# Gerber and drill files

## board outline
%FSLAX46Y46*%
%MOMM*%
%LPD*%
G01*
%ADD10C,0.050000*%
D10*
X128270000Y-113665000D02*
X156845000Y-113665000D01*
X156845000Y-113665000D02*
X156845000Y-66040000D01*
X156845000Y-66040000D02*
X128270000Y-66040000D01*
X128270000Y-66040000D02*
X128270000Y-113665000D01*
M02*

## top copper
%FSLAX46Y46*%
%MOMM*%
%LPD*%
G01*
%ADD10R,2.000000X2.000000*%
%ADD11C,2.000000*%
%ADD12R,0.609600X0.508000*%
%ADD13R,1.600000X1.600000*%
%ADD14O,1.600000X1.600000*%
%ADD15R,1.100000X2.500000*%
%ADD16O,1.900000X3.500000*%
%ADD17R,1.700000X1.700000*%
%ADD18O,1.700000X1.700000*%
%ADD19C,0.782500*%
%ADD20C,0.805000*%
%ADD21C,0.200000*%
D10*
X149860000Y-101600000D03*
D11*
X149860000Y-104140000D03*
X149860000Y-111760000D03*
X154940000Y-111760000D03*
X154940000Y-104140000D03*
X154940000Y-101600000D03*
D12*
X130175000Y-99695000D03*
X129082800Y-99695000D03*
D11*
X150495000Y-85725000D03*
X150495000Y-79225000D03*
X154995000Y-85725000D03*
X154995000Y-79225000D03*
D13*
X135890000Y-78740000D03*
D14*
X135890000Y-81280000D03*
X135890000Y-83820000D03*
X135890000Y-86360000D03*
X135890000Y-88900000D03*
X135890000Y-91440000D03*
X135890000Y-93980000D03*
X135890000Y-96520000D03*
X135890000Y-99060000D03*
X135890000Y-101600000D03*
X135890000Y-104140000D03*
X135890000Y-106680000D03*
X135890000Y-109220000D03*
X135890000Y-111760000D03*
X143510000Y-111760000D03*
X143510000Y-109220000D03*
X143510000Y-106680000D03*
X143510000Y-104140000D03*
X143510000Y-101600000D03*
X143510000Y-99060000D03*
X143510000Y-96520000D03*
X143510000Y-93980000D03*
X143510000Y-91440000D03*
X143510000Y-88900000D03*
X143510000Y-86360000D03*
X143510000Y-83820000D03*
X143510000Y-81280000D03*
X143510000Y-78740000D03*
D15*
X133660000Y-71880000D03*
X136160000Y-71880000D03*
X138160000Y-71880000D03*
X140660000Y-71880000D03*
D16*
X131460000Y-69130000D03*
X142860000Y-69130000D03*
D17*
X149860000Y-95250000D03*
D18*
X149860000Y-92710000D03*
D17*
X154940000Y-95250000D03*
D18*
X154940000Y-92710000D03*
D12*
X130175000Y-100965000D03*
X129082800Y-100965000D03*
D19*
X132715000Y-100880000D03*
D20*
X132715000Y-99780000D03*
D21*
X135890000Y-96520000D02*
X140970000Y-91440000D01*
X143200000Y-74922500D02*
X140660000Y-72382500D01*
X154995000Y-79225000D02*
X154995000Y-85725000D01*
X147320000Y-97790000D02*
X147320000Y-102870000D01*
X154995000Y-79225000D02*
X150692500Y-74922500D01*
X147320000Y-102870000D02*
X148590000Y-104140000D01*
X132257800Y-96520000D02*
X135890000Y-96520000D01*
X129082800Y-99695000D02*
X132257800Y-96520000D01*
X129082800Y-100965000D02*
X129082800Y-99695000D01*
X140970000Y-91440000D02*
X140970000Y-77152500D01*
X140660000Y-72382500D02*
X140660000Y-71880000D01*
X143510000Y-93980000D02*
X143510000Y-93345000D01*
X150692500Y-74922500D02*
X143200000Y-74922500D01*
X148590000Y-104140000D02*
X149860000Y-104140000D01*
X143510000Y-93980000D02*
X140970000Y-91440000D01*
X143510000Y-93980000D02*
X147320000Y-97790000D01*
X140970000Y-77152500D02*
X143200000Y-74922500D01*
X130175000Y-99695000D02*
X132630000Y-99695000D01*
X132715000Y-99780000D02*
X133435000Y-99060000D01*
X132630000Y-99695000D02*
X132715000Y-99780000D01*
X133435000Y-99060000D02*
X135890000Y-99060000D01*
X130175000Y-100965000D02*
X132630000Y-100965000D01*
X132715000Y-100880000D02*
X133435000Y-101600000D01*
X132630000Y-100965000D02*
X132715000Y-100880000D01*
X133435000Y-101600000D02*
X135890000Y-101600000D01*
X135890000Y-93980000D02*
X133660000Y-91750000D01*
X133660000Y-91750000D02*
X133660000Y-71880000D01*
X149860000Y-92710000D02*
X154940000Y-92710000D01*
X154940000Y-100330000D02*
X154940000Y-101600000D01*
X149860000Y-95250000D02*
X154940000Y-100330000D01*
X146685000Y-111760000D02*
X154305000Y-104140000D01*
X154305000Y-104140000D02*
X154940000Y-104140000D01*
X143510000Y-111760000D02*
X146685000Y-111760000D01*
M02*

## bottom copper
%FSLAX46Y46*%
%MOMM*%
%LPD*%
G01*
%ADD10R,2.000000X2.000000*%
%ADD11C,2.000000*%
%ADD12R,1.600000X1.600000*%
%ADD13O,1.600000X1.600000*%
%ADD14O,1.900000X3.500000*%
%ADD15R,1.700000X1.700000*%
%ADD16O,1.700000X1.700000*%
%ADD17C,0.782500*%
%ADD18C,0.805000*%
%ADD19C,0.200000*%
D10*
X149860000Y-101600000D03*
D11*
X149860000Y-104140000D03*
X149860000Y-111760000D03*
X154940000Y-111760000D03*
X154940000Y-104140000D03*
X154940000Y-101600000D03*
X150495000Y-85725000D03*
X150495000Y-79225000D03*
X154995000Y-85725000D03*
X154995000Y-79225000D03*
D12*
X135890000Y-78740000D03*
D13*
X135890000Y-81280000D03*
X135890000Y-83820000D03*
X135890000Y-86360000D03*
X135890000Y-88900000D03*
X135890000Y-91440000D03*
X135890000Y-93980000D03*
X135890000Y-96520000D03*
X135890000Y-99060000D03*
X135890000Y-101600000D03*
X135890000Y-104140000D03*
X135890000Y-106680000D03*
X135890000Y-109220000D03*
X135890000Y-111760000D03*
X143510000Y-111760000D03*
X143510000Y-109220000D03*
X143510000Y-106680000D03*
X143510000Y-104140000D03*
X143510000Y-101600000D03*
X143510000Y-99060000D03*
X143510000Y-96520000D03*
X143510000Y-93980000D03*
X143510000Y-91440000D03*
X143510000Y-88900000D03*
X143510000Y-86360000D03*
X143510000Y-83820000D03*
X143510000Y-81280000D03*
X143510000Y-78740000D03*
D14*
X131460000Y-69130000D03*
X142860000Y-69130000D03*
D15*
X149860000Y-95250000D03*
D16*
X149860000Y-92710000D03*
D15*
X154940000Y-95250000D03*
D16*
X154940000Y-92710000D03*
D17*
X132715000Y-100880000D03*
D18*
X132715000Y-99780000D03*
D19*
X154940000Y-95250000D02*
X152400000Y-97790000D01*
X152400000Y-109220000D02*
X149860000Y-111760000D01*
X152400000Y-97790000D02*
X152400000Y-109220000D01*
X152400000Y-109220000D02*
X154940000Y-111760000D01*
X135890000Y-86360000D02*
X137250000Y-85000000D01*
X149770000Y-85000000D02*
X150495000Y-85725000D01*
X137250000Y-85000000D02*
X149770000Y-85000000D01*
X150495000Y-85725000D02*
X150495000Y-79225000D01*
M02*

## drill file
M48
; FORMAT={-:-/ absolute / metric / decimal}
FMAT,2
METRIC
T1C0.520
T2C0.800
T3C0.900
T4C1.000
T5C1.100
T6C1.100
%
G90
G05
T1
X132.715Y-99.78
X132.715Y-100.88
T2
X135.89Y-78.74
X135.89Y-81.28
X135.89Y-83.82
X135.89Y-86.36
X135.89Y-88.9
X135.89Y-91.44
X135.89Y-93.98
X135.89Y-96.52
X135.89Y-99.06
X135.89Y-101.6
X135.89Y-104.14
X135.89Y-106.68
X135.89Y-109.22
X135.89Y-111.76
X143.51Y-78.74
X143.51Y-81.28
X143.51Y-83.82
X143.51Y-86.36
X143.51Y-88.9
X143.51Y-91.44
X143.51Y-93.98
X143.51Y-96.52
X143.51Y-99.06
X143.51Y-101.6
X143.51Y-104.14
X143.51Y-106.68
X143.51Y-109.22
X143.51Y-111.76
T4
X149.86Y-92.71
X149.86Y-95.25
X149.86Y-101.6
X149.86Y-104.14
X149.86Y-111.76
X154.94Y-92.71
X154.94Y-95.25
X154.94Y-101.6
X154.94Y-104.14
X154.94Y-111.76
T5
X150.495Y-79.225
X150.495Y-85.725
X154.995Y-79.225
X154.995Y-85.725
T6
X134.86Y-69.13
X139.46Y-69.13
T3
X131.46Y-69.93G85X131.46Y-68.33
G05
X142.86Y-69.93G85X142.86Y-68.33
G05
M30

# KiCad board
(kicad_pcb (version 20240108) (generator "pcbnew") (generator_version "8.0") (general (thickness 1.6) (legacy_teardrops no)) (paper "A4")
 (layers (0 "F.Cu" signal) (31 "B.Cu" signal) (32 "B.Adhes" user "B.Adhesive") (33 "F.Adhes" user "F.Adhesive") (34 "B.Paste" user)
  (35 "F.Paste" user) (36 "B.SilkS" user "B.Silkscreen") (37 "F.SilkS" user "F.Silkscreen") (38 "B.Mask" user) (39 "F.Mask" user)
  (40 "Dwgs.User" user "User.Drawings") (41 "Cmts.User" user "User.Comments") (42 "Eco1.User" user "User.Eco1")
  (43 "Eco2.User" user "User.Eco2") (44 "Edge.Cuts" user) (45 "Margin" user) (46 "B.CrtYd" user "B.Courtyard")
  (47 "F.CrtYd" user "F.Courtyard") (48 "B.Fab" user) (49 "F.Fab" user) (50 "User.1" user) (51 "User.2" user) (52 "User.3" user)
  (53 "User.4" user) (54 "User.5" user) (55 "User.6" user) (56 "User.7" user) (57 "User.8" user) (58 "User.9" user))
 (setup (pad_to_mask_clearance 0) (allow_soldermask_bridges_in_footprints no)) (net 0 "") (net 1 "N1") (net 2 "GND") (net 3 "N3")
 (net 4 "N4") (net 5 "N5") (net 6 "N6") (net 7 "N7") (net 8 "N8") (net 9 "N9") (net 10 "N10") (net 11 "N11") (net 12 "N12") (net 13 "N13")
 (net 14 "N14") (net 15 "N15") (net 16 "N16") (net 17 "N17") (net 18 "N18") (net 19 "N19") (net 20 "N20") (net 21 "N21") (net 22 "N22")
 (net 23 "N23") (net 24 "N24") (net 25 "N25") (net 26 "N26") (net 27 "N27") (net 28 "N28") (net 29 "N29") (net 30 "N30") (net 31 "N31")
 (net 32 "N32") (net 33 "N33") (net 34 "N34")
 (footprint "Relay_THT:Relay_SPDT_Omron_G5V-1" (layer "F.Cu") (at 149.86 101.6)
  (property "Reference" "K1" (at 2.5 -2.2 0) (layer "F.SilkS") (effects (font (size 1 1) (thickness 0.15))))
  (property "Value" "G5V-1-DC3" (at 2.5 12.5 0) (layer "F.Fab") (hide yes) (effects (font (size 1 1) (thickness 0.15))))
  (pad "1" thru_hole rect (at 0 0) (size 2 2) (drill 1) (layers "*.Cu" "*.Mask") (remove_unused_layers no) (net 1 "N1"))
  (pad "2" thru_hole circle (at 0 2.54) (size 2 2) (drill 1) (layers "*.Cu" "*.Mask") (remove_unused_layers no) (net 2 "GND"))
  (pad "5" thru_hole circle (at 0 10.16) (size 2 2) (drill 1) (layers "*.Cu" "*.Mask") (remove_unused_layers no) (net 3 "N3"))
  (pad "6" thru_hole circle (at 5.08 10.16) (size 2 2) (drill 1) (layers "*.Cu" "*.Mask") (remove_unused_layers no) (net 3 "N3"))
  (pad "9" thru_hole circle (at 5.08 2.54) (size 2 2) (drill 1) (layers "*.Cu" "*.Mask") (remove_unused_layers no) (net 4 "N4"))
  (pad "10" thru_hole circle (at 5.08 0) (size 2 2) (drill 1) (layers "*.Cu" "*.Mask") (remove_unused_layers no) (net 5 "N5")))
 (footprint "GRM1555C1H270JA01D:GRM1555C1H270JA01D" (layer "F.Cu") (at 129.6289 99.695 180)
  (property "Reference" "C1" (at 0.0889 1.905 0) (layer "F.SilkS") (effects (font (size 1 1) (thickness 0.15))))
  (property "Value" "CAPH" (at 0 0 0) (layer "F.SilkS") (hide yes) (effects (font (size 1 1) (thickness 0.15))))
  (pad "1" smd rect (at -0.5461 0 180) (size 0.6096 0.508) (layers "F.Cu" "F.Paste" "F.Mask") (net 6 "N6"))
  (pad "2" smd rect (at 0.5461 0 180) (size 0.6096 0.508) (layers "F.Cu" "F.Paste" "F.Mask") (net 2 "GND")))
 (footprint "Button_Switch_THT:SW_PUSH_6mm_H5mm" (layer "F.Cu") (at 150.495 85.725 90)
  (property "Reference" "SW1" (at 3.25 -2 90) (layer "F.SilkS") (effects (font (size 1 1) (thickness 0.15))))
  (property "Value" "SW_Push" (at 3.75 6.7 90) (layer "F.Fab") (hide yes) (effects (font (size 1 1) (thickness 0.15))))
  (pad "1" thru_hole circle (at 0 0 180) (size 2 2) (drill 1.1) (layers "*.Cu" "*.Mask") (remove_unused_layers no) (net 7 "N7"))
  (pad "1" thru_hole circle (at 6.5 0 180) (size 2 2) (drill 1.1) (layers "*.Cu" "*.Mask") (remove_unused_layers no) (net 7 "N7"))
  (pad "2" thru_hole circle (at 0 4.5 180) (size 2 2) (drill 1.1) (layers "*.Cu" "*.Mask") (remove_unused_layers no) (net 2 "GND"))
  (pad "2" thru_hole circle (at 6.5 4.5 180) (size 2 2) (drill 1.1) (layers "*.Cu" "*.Mask") (remove_unused_layers no) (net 2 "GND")))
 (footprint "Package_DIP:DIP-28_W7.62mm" (layer "F.Cu") (at 135.89 78.74)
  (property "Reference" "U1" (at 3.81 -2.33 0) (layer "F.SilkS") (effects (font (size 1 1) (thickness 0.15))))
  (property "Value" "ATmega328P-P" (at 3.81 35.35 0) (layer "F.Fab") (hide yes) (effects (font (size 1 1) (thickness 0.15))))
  (pad "1" thru_hole rect (at 0 0) (size 1.6 1.6) (drill 0.8) (layers "*.Cu" "*.Mask") (remove_unused_layers no) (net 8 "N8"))
  (pad "2" thru_hole oval (at 0 2.54) (size 1.6 1.6) (drill 0.8) (layers "*.Cu" "*.Mask") (remove_unused_layers no) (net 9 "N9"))
  (pad "3" thru_hole oval (at 0 5.08) (size 1.6 1.6) (drill 0.8) (layers "*.Cu" "*.Mask") (remove_unused_layers no) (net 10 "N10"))
  (pad "4" thru_hole oval (at 0 7.62) (size 1.6 1.6) (drill 0.8) (layers "*.Cu" "*.Mask") (remove_unused_layers no) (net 7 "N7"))
  (pad "5" thru_hole oval (at 0 10.16) (size 1.6 1.6) (drill 0.8) (layers "*.Cu" "*.Mask") (remove_unused_layers no) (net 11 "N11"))
  (pad "6" thru_hole oval (at 0 12.7) (size 1.6 1.6) (drill 0.8) (layers "*.Cu" "*.Mask") (remove_unused_layers no) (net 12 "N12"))
  (pad "7" thru_hole oval (at 0 15.24) (size 1.6 1.6) (drill 0.8) (layers "*.Cu" "*.Mask") (remove_unused_layers no) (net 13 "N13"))
  (pad "8" thru_hole oval (at 0 17.78) (size 1.6 1.6) (drill 0.8) (layers "*.Cu" "*.Mask") (remove_unused_layers no) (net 2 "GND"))
  (pad "9" thru_hole oval (at 0 20.32) (size 1.6 1.6) (drill 0.8) (layers "*.Cu" "*.Mask") (remove_unused_layers no) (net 6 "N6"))
  (pad "10" thru_hole oval (at 0 22.86) (size 1.6 1.6) (drill 0.8) (layers "*.Cu" "*.Mask") (remove_unused_layers no) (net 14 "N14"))
  (pad "11" thru_hole oval (at 0 25.4) (size 1.6 1.6) (drill 0.8) (layers "*.Cu" "*.Mask") (remove_unused_layers no) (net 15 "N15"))
  (pad "12" thru_hole oval (at 0 27.94) (size 1.6 1.6) (drill 0.8) (layers "*.Cu" "*.Mask") (remove_unused_layers no) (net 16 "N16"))
  (pad "13" thru_hole oval (at 0 30.48) (size 1.6 1.6) (drill 0.8) (layers "*.Cu" "*.Mask") (remove_unused_layers no) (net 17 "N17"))
  (pad "14" thru_hole oval (at 0 33.02) (size 1.6 1.6) (drill 0.8) (layers "*.Cu" "*.Mask") (remove_unused_layers no) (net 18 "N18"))
  (pad "15" thru_hole oval (at 7.62 33.02) (size 1.6 1.6) (drill 0.8) (layers "*.Cu" "*.Mask") (remove_unused_layers no) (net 4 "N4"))
  (pad "16" thru_hole oval (at 7.62 30.48) (size 1.6 1.6) (drill 0.8) (layers "*.Cu" "*.Mask") (remove_unused_layers no) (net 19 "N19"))
  (pad "17" thru_hole oval (at 7.62 27.94) (size 1.6 1.6) (drill 0.8) (layers "*.Cu" "*.Mask") (remove_unused_layers no) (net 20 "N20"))
  (pad "18" thru_hole oval (at 7.62 25.4) (size 1.6 1.6) (drill 0.8) (layers "*.Cu" "*.Mask") (remove_unused_layers no) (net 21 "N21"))
  (pad "19" thru_hole oval (at 7.62 22.86) (size 1.6 1.6) (drill 0.8) (layers "*.Cu" "*.Mask") (remove_unused_layers no) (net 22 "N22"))
  (pad "20" thru_hole oval (at 7.62 20.32) (size 1.6 1.6) (drill 0.8) (layers "*.Cu" "*.Mask") (remove_unused_layers no) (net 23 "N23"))
  (pad "21" thru_hole oval (at 7.62 17.78) (size 1.6 1.6) (drill 0.8) (layers "*.Cu" "*.Mask") (remove_unused_layers no) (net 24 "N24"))
  (pad "22" thru_hole oval (at 7.62 15.24) (size 1.6 1.6) (drill 0.8) (layers "*.Cu" "*.Mask") (remove_unused_layers no) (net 2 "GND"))
  (pad "23" thru_hole oval (at 7.62 12.7) (size 1.6 1.6) (drill 0.8) (layers "*.Cu" "*.Mask") (remove_unused_layers no) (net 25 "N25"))
  (pad "24" thru_hole oval (at 7.62 10.16) (size 1.6 1.6) (drill 0.8) (layers "*.Cu" "*.Mask") (remove_unused_layers no) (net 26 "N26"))
  (pad "25" thru_hole oval (at 7.62 7.62) (size 1.6 1.6) (drill 0.8) (layers "*.Cu" "*.Mask") (remove_unused_layers no) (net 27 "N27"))
  (pad "26" thru_hole oval (at 7.62 5.08) (size 1.6 1.6) (drill 0.8) (layers "*.Cu" "*.Mask") (remove_unused_layers no) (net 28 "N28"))
  (pad "27" thru_hole oval (at 7.62 2.54) (size 1.6 1.6) (drill 0.8) (layers "*.Cu" "*.Mask") (remove_unused_layers no) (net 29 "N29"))
  (pad "28" thru_hole oval (at 7.62 0) (size 1.6 1.6) (drill 0.8) (layers "*.Cu" "*.Mask") (remove_unused_layers no) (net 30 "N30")))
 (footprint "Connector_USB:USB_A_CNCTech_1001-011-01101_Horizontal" (layer "F.Cu") (at 137.16 62.23 90)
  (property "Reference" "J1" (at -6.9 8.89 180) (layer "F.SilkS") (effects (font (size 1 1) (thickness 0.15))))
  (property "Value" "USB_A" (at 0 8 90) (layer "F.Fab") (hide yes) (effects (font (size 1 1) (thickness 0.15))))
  (pad "" np_thru_hole circle (at -6.9 -2.3 90) (size 1.1 1.1) (drill 1.1) (layers "*.Cu" "*.Mask"))
  (pad "" np_thru_hole circle (at -6.9 2.3 90) (size 1.1 1.1) (drill 1.1) (layers "*.Cu" "*.Mask"))
  (pad "1" smd rect (at -9.65 -3.5 90) (size 2.5 1.1) (layers "F.Cu" "F.Paste" "F.Mask") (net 13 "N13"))
  (pad "2" smd rect (at -9.65 -1 90) (size 2.5 1.1) (layers "F.Cu" "F.Paste" "F.Mask") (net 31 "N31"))
  (pad "3" smd rect (at -9.65 1 90) (size 2.5 1.1) (layers "F.Cu" "F.Paste" "F.Mask") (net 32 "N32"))
  (pad "4" smd rect (at -9.65 3.5 90) (size 2.5 1.1) (layers "F.Cu" "F.Paste" "F.Mask") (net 2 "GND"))
  (pad "5" thru_hole oval (at -6.9 -5.7 90) (size 3.5 1.9) (drill oval 2.5 0.9) (layers "*.Cu" "*.Mask") (remove_unused_layers no)
   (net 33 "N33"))
  (pad "5" thru_hole oval (at -6.9 5.7 90) (size 3.5 1.9) (drill oval 2.5 0.9) (layers "*.Cu" "*.Mask") (remove_unused_layers no)
   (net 33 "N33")))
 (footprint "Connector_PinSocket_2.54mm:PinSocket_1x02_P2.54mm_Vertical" (layer "F.Cu") (at 149.86 95.25 180)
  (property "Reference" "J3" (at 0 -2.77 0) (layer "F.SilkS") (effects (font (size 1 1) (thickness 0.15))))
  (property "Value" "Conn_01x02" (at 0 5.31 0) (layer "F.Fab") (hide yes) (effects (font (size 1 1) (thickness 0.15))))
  (pad "1" thru_hole rect (at 0 0 180) (size 1.7 1.7) (drill 1) (layers "*.Cu" "*.Mask") (remove_unused_layers no) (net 5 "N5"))
  (pad "2" thru_hole oval (at 0 2.54 180) (size 1.7 1.7) (drill 1) (layers "*.Cu" "*.Mask") (remove_unused_layers no) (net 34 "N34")))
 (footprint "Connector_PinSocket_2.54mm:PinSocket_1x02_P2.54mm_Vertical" (layer "F.Cu") (at 154.94 95.25 180)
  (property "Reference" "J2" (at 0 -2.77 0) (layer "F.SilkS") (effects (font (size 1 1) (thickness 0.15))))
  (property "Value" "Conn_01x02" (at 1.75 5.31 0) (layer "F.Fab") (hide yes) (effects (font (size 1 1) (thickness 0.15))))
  (pad "1" thru_hole rect (at 0 0 180) (size 1.7 1.7) (drill 1) (layers "*.Cu" "*.Mask") (remove_unused_layers no) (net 3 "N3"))
  (pad "2" thru_hole oval (at 0 2.54 180) (size 1.7 1.7) (drill 1) (layers "*.Cu" "*.Mask") (remove_unused_layers no) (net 34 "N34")))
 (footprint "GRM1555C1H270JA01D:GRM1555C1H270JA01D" (layer "F.Cu") (at 129.6289 100.965 180)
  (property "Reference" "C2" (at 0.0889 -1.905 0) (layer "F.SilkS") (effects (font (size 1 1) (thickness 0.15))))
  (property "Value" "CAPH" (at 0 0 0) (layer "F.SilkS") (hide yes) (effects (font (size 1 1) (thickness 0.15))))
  (pad "1" smd rect (at -0.5461 0 180) (size 0.6096 0.508) (layers "F.Cu" "F.Paste" "F.Mask") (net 14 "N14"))
  (pad "2" smd rect (at 0.5461 0 180) (size 0.6096 0.508) (layers "F.Cu" "F.Paste" "F.Mask") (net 2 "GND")))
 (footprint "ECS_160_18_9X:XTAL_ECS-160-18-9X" (layer "F.Cu") (at 132.715 100.33 90)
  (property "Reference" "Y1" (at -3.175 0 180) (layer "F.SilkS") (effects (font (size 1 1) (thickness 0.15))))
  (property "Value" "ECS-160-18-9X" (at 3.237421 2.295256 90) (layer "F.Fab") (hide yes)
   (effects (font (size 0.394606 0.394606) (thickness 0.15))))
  (pad "1" thru_hole circle (at -0.55 0 90) (size 0.7825 0.7825) (drill 0.52) (layers "*.Cu" "*.Mask") (remove_unused_layers no)
   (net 14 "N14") (solder_mask_margin 0.102))
  (pad "2" thru_hole circle (at 0.55 0 90) (size 0.805 0.805) (drill 0.52) (layers "*.Cu" "*.Mask") (remove_unused_layers no) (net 6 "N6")
   (solder_mask_margin 0.102)))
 (gr_line (start 128.27 113.665) (end 156.845 113.665) (stroke (width 0.05) (type default)) (layer "Edge.Cuts"))
 (gr_line (start 156.845 113.665) (end 156.845 66.04) (stroke (width 0.05) (type default)) (layer "Edge.Cuts"))
 (gr_line (start 156.845 66.04) (end 128.27 66.04) (stroke (width 0.05) (type default)) (layer "Edge.Cuts"))
 (gr_line (start 128.27 66.04) (end 128.27 113.665) (stroke (width 0.05) (type default)) (layer "Edge.Cuts"))
 (segment (start 135.89 96.52) (end 140.97 91.44) (width 0.2) (layer "F.Cu") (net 2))
 (segment (start 143.2 74.9225) (end 140.66 72.3825) (width 0.2) (layer "F.Cu") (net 2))
 (segment (start 154.995 79.225) (end 154.995 85.725) (width 0.2) (layer "F.Cu") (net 2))
 (segment (start 147.32 97.79) (end 147.32 102.87) (width 0.2) (layer "F.Cu") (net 2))
 (segment (start 154.995 79.225) (end 150.6925 74.9225) (width 0.2) (layer "F.Cu") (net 2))
 (segment (start 147.32 102.87) (end 148.59 104.14) (width 0.2) (layer "F.Cu") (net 2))
 (segment (start 132.2578 96.52) (end 135.89 96.52) (width 0.2) (layer "F.Cu") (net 2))
 (segment (start 129.0828 99.695) (end 132.2578 96.52) (width 0.2) (layer "F.Cu") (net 2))
 (segment (start 129.0828 100.965) (end 129.0828 99.695) (width 0.2) (layer "F.Cu") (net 2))
 (segment (start 140.97 91.44) (end 140.97 77.1525) (width 0.2) (layer "F.Cu") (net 2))
 (segment (start 140.66 72.3825) (end 140.66 71.88) (width 0.2) (layer "F.Cu") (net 2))
 (segment (start 143.51 93.98) (end 143.51 93.345) (width 0.2) (layer "F.Cu") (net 2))
 (segment (start 150.6925 74.9225) (end 143.2 74.9225) (width 0.2) (layer "F.Cu") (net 2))
 (segment (start 148.59 104.14) (end 149.86 104.14) (width 0.2) (layer "F.Cu") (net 2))
 (segment (start 143.51 93.98) (end 140.97 91.44) (width 0.2) (layer "F.Cu") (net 2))
 (segment (start 143.51 93.98) (end 147.32 97.79) (width 0.2) (layer "F.Cu") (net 2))
 (segment (start 140.97 77.1525) (end 143.2 74.9225) (width 0.2) (layer "F.Cu") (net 2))
 (segment (start 130.175 99.695) (end 132.63 99.695) (width 0.2) (layer "F.Cu") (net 6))
 (segment (start 132.715 99.78) (end 133.435 99.06) (width 0.2) (layer "F.Cu") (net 6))
 (segment (start 132.63 99.695) (end 132.715 99.78) (width 0.2) (layer "F.Cu") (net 6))
 (segment (start 133.435 99.06) (end 135.89 99.06) (width 0.2) (layer "F.Cu") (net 6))
 (segment (start 130.175 100.965) (end 132.63 100.965) (width 0.2) (layer "F.Cu") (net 14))
 (segment (start 132.715 100.88) (end 133.435 101.6) (width 0.2) (layer "F.Cu") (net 14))
 (segment (start 132.63 100.965) (end 132.715 100.88) (width 0.2) (layer "F.Cu") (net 14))
 (segment (start 133.435 101.6) (end 135.89 101.6) (width 0.2) (layer "F.Cu") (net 14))
 (segment (start 135.89 93.98) (end 133.66 91.75) (width 0.2) (layer "F.Cu") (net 13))
 (segment (start 133.66 91.75) (end 133.66 71.88) (width 0.2) (layer "F.Cu") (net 13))
 (segment (start 154.94 95.25) (end 152.4 97.79) (width 0.2) (layer "B.Cu") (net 3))
 (segment (start 152.4 109.22) (end 149.86 111.76) (width 0.2) (layer "B.Cu") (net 3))
 (segment (start 152.4 97.79) (end 152.4 109.22) (width 0.2) (layer "B.Cu") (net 3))
 (segment (start 152.4 109.22) (end 154.94 111.76) (width 0.2) (layer "B.Cu") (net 3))
 (segment (start 149.86 92.71) (end 154.94 92.71) (width 0.2) (layer "F.Cu") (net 34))
 (segment (start 154.94 100.33) (end 154.94 101.6) (width 0.2) (layer "F.Cu") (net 5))
 (segment (start 149.86 95.25) (end 154.94 100.33) (width 0.2) (layer "F.Cu") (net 5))
 (segment (start 146.685 111.76) (end 154.305 104.14) (width 0.2) (layer "F.Cu") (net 4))
 (segment (start 154.305 104.14) (end 154.94 104.14) (width 0.2) (layer "F.Cu") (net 4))
 (segment (start 143.51 111.76) (end 146.685 111.76) (width 0.2) (layer "F.Cu") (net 4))
 (segment (start 135.89 86.36) (end 137.25 85) (width 0.2) (layer "B.Cu") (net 7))
 (segment (start 149.77 85) (end 150.495 85.725) (width 0.2) (layer "B.Cu") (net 7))
 (segment (start 137.25 85) (end 149.77 85) (width 0.2) (layer "B.Cu") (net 7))
 (segment (start 150.495 85.725) (end 150.495 79.225) (width 0.2) (layer "B.Cu") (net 7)))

